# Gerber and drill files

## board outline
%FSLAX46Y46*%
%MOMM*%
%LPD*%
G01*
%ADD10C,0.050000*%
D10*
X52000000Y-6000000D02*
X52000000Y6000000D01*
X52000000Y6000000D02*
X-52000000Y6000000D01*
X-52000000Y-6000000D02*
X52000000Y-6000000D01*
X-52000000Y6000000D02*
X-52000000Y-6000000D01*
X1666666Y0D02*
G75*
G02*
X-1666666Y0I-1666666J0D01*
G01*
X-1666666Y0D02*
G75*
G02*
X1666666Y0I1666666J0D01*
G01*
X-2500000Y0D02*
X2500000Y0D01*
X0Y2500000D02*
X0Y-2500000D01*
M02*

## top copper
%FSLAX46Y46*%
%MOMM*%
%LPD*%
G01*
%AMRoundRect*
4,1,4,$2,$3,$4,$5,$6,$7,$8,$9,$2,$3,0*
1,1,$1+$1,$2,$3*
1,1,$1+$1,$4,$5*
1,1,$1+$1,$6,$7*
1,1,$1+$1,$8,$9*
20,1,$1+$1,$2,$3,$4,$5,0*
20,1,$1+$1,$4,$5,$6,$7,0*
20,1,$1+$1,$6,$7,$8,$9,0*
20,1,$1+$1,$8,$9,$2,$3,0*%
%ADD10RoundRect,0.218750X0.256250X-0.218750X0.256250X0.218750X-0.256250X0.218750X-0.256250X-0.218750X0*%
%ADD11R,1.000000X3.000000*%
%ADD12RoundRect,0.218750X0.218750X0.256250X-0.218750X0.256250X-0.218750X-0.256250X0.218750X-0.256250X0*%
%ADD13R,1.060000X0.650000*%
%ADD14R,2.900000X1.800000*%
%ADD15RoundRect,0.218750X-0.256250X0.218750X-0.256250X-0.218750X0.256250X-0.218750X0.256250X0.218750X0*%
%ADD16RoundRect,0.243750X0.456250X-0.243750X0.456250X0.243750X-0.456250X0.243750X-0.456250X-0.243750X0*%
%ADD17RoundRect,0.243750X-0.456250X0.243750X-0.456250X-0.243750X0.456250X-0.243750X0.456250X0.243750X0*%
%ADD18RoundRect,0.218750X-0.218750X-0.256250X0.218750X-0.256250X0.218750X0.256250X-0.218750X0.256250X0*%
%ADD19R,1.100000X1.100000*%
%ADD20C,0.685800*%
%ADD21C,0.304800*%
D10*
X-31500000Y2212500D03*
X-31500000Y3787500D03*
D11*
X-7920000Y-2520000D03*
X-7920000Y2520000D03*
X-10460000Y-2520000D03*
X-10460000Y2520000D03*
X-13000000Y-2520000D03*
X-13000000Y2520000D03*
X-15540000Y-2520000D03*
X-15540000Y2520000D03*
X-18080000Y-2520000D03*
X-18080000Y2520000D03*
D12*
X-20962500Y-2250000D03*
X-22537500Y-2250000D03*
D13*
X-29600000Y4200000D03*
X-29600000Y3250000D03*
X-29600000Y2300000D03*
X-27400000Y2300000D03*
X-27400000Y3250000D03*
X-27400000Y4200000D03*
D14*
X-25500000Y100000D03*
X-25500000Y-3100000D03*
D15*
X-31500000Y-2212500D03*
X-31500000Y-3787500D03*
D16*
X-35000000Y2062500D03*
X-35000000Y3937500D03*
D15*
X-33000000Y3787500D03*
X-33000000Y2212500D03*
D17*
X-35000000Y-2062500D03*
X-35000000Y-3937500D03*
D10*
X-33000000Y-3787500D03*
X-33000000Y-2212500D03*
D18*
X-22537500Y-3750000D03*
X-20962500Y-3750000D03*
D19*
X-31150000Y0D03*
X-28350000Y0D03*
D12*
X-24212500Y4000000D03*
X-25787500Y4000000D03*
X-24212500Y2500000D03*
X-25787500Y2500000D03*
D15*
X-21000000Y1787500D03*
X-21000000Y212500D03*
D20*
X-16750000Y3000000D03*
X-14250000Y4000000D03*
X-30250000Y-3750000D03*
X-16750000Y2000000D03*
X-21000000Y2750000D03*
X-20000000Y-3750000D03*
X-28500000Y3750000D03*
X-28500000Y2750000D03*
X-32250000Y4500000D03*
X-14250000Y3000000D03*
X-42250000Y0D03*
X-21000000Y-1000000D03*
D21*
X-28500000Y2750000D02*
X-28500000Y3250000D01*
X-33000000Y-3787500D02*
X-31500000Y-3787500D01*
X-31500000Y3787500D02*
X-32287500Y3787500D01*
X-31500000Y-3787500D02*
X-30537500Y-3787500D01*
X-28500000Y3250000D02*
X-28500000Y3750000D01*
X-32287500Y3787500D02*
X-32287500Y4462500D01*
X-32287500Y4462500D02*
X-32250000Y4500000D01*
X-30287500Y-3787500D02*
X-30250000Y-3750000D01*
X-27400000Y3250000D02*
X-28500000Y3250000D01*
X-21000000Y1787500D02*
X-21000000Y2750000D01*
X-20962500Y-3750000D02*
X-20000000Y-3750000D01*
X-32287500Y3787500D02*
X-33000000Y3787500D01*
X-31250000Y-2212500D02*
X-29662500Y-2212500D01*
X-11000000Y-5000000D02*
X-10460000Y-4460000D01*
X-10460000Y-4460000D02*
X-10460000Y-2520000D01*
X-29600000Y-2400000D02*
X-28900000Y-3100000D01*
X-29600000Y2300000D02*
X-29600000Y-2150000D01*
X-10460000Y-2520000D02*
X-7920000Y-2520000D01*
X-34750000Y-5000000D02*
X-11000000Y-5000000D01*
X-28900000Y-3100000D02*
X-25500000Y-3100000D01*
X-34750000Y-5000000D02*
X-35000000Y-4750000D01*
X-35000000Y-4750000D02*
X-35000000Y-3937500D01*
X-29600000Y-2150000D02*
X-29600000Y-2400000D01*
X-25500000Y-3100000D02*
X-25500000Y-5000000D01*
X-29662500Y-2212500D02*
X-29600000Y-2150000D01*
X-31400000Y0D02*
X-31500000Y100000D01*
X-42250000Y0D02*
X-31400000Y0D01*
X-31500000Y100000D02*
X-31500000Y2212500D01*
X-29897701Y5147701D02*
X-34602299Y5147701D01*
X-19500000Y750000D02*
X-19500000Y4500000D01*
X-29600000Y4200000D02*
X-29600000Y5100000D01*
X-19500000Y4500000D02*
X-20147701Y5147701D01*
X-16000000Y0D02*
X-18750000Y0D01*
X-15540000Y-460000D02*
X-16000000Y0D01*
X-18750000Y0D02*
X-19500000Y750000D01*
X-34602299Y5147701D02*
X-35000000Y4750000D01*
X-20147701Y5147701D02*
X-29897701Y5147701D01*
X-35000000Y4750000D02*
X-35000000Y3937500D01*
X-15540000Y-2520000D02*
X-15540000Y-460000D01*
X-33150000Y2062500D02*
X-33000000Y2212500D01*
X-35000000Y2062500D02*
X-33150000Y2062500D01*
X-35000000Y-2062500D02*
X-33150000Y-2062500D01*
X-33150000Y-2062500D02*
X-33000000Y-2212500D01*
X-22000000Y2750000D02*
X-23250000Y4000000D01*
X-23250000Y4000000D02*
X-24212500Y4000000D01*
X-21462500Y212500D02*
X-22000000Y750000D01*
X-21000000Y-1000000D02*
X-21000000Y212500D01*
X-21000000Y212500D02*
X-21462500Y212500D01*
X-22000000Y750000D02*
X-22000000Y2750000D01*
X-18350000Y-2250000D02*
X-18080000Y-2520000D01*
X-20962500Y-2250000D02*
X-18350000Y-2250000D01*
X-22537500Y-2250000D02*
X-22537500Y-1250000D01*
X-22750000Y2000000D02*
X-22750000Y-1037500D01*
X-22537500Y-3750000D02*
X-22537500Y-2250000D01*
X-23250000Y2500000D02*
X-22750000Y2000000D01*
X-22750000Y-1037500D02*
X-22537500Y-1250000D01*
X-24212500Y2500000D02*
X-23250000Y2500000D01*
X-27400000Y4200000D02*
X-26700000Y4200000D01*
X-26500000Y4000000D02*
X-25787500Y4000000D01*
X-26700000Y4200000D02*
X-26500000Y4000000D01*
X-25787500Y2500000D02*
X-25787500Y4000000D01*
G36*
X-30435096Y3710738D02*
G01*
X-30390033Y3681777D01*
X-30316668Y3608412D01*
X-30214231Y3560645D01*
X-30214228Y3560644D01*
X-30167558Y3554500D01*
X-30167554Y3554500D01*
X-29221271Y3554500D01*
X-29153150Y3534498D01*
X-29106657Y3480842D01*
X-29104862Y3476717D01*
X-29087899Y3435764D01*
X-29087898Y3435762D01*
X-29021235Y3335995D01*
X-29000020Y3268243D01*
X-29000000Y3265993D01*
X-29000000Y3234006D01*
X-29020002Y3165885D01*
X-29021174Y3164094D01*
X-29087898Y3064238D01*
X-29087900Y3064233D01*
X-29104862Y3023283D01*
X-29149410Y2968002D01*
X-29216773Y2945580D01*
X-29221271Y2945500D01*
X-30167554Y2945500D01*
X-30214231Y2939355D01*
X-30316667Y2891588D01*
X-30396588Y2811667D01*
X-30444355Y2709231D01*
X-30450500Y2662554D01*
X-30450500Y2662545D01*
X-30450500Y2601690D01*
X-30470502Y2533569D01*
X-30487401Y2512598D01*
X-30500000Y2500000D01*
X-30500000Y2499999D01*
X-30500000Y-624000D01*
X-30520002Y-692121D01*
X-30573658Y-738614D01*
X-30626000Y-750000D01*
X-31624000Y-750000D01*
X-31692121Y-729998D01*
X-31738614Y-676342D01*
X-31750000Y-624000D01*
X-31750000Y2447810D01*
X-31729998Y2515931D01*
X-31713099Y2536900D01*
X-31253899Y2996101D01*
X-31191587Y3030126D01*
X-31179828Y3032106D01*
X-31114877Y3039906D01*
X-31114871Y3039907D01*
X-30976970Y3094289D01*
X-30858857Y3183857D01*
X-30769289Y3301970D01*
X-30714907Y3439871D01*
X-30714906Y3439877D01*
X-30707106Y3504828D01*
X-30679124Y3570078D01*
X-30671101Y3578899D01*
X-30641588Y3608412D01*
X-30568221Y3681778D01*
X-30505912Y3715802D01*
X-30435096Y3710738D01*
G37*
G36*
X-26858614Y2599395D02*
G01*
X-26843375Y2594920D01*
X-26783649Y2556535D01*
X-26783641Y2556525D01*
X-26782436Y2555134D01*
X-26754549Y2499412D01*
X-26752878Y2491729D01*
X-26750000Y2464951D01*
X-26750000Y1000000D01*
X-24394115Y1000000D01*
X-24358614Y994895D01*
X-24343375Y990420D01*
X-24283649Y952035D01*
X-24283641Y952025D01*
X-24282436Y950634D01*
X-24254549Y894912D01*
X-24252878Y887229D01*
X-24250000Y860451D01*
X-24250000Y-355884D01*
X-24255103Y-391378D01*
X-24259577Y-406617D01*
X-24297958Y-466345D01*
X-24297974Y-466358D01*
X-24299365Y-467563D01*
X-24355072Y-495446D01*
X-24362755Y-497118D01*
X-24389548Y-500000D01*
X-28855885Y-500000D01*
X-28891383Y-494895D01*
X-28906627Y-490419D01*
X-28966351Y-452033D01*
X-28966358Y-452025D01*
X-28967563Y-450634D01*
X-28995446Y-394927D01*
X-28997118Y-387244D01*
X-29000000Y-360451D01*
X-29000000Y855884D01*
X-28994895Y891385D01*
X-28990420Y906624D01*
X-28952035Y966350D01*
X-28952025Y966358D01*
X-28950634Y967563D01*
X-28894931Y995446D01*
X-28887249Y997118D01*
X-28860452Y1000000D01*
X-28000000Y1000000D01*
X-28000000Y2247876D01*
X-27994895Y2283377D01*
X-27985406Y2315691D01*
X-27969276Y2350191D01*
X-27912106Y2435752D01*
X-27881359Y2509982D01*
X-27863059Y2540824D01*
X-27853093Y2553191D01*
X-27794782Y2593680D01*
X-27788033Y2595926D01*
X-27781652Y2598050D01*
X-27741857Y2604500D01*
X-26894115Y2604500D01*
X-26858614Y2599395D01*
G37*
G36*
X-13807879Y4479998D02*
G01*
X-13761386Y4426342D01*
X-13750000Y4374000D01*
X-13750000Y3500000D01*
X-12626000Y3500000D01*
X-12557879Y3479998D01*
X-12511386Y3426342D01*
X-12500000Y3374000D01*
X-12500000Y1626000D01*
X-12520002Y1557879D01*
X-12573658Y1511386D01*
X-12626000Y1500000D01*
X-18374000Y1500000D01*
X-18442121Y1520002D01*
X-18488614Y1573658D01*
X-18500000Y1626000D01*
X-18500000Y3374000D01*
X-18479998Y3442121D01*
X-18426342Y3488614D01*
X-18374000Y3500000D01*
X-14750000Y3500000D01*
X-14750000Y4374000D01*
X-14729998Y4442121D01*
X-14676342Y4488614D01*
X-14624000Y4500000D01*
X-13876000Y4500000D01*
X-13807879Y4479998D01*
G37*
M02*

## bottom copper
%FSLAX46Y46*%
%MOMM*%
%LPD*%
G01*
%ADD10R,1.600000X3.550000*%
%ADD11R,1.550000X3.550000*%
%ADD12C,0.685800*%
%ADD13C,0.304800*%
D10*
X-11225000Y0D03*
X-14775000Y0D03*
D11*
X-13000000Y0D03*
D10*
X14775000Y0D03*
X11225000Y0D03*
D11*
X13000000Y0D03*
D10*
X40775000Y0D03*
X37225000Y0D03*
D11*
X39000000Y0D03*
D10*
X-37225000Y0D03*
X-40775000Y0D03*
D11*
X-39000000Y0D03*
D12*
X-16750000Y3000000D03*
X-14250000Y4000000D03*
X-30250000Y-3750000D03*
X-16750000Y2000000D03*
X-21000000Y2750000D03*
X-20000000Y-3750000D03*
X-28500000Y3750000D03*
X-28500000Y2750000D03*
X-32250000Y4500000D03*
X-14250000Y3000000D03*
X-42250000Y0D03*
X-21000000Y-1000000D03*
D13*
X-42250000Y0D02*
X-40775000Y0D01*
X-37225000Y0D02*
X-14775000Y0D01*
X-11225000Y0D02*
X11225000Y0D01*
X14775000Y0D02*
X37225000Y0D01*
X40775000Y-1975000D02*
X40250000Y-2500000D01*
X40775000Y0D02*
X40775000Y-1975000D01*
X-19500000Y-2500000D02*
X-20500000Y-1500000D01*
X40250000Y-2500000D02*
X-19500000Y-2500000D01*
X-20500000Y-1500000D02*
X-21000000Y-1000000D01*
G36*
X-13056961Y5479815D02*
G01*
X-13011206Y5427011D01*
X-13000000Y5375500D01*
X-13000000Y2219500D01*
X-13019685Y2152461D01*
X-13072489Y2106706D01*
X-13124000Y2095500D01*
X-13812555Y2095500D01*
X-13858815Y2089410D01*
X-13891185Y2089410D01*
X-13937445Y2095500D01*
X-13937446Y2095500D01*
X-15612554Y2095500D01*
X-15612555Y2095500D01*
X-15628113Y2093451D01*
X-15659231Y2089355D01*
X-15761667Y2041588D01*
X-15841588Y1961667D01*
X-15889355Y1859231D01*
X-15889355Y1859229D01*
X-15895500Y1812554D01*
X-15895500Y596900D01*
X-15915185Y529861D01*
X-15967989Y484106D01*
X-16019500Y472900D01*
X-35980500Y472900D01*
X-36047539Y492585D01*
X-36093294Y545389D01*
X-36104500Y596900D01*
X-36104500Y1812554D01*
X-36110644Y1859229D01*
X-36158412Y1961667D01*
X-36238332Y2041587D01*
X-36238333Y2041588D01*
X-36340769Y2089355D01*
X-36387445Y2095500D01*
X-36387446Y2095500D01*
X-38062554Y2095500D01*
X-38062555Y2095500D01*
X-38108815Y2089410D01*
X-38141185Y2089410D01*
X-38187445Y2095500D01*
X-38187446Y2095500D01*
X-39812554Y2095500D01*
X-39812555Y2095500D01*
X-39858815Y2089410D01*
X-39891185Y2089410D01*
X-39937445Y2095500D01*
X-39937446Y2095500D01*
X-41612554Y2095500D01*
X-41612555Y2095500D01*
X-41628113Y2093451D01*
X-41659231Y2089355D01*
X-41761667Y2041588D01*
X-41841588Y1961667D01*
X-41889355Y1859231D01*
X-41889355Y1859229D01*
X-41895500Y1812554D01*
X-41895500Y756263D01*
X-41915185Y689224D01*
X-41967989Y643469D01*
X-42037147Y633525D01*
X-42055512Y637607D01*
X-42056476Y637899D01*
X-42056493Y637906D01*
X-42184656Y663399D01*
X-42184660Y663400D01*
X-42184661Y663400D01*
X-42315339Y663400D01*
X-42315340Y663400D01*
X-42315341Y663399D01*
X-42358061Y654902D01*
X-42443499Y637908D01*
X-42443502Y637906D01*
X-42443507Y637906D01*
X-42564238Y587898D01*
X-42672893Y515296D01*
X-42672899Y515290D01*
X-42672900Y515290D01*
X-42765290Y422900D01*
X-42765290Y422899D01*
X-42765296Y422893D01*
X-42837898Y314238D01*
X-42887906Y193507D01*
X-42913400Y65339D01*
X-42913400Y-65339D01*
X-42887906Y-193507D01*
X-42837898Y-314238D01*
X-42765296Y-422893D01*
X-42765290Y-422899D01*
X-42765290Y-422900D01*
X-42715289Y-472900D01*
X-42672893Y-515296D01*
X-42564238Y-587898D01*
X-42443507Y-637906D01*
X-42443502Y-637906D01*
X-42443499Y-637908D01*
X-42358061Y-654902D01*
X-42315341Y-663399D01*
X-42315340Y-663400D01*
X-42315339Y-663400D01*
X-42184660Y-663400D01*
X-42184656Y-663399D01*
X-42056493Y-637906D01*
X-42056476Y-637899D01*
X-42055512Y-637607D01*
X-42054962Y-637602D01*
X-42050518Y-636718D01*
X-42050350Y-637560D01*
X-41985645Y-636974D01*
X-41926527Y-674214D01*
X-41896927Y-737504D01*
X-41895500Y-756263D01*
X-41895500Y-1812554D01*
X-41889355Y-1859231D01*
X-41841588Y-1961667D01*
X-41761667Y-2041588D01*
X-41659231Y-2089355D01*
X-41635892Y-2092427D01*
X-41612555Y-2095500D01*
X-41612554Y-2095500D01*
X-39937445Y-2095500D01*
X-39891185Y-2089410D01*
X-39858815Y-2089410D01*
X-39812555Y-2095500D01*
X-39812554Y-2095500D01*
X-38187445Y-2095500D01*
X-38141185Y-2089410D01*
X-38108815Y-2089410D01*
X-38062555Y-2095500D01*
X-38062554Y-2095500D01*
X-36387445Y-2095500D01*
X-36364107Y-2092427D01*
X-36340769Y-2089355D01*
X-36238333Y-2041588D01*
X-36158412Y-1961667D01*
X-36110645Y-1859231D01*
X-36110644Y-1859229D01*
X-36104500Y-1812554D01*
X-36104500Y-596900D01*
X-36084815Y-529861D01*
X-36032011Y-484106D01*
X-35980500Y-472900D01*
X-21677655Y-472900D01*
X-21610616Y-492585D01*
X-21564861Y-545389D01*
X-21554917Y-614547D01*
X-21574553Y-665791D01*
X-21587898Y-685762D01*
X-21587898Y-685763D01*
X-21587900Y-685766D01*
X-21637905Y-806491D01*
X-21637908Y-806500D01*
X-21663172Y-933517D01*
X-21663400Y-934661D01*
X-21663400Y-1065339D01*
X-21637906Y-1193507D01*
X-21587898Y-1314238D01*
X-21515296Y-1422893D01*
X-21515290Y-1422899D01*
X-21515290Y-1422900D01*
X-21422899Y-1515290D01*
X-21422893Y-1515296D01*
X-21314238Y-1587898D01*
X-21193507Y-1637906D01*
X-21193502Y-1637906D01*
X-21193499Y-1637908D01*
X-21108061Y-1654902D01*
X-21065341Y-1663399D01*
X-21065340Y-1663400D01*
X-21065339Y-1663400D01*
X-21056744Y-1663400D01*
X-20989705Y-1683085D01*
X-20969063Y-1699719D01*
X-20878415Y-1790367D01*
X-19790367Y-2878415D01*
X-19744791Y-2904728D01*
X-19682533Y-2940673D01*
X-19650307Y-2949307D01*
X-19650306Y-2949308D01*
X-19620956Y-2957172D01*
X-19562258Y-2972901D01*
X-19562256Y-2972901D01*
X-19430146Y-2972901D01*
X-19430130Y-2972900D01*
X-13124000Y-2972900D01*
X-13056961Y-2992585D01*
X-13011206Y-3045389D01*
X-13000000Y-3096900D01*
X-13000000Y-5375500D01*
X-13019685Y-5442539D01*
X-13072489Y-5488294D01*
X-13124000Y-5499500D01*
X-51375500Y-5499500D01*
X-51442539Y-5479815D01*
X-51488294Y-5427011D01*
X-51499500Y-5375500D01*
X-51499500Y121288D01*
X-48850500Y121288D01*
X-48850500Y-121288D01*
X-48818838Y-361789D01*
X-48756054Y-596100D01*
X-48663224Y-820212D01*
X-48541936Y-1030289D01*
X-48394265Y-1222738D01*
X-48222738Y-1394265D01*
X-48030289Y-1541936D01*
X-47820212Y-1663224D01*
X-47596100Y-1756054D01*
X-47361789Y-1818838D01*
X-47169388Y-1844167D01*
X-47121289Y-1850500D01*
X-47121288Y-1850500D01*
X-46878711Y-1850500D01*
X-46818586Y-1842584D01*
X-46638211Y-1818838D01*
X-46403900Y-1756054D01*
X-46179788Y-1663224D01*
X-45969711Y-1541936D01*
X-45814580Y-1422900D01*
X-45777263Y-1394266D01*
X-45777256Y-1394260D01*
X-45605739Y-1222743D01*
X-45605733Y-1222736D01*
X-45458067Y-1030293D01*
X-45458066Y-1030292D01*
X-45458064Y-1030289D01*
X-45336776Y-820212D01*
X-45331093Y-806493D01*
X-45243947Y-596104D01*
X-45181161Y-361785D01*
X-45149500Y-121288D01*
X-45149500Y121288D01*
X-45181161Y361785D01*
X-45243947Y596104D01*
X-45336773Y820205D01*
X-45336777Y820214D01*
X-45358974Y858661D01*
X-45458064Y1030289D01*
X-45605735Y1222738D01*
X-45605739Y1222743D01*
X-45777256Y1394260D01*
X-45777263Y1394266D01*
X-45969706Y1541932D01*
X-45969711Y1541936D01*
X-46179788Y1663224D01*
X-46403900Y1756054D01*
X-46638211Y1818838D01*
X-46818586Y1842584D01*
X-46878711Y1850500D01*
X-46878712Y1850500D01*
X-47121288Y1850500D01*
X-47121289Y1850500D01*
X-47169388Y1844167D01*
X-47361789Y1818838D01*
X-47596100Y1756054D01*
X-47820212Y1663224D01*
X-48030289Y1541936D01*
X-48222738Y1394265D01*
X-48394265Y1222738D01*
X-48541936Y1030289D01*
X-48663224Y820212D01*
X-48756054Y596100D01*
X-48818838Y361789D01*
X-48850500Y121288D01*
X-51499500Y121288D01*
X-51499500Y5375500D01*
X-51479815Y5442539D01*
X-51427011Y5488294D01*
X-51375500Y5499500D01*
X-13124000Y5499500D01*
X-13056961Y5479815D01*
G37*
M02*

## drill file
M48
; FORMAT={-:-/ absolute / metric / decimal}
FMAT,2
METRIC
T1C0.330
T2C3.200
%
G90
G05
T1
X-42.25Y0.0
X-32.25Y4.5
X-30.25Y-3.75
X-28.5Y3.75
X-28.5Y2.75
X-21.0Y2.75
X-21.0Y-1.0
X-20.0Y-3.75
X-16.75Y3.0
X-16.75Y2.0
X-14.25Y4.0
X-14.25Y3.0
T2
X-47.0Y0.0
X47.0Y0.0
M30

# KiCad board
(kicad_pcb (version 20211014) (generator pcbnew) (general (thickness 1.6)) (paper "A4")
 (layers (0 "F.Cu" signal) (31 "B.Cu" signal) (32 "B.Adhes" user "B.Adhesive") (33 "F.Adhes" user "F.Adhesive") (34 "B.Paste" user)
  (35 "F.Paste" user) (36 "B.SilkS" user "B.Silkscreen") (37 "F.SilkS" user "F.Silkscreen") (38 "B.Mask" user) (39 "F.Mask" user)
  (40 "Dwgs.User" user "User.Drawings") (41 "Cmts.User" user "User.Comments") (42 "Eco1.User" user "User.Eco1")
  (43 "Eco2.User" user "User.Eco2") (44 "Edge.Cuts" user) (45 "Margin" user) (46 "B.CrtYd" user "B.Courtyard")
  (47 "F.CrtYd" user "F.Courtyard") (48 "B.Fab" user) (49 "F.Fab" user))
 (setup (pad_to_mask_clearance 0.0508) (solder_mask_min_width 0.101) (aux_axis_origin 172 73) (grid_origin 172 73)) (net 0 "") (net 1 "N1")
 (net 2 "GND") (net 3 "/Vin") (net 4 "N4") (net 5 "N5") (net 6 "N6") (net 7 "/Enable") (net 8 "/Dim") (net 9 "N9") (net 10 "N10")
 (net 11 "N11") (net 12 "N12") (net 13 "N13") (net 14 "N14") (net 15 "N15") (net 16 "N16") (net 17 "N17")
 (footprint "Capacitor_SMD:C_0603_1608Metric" (layer "F.Cu") (at -31.5 -3 90)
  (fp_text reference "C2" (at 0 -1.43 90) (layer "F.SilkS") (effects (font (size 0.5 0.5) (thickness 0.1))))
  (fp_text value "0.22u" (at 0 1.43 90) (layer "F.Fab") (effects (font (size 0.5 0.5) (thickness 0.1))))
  (pad "1" smd roundrect locked (at -0.7875 0 90) (size 0.875 0.95) (layers "F.Cu" "F.Paste" "F.Mask") (roundrect_rratio 0.25) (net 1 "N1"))
  (pad "2" smd roundrect locked (at 0.7875 0 90) (size 0.875 0.95) (layers "F.Cu" "F.Paste" "F.Mask") (roundrect_rratio 0.25) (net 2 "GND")))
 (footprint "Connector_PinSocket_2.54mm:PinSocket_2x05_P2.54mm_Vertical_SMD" (layer "F.Cu") (at -13 0 -90)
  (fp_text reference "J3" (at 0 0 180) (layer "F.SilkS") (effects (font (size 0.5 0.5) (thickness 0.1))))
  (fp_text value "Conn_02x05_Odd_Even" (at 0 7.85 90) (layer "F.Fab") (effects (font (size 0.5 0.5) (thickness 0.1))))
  (pad "1" smd rect locked (at 2.52 -5.08 270) (size 3 1) (layers "F.Cu" "F.Paste" "F.Mask") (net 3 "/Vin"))
  (pad "2" smd rect locked (at -2.52 -5.08 270) (size 3 1) (layers "F.Cu" "F.Paste" "F.Mask") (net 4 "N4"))
  (pad "3" smd rect locked (at 2.52 -2.54 270) (size 3 1) (layers "F.Cu" "F.Paste" "F.Mask") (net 3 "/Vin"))
  (pad "4" smd rect locked (at -2.52 -2.54 270) (size 3 1) (layers "F.Cu" "F.Paste" "F.Mask") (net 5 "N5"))
  (pad "5" smd rect locked (at 2.52 0 270) (size 3 1) (layers "F.Cu" "F.Paste" "F.Mask") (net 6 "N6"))
  (pad "6" smd rect locked (at -2.52 0 270) (size 3 1) (layers "F.Cu" "F.Paste" "F.Mask") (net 2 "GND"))
  (pad "7" smd rect locked (at 2.52 2.54 270) (size 3 1) (layers "F.Cu" "F.Paste" "F.Mask") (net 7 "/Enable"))
  (pad "8" smd rect locked (at -2.52 2.54 270) (size 3 1) (layers "F.Cu" "F.Paste" "F.Mask") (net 2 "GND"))
  (pad "9" smd rect locked (at 2.52 5.08 270) (size 3 1) (layers "F.Cu" "F.Paste" "F.Mask") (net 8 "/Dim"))
  (pad "10" smd rect locked (at -2.52 5.08 270) (size 3 1) (layers "F.Cu" "F.Paste" "F.Mask") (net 2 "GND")))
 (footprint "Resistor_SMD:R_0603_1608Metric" (layer "F.Cu") (at -21.75 2.25 180)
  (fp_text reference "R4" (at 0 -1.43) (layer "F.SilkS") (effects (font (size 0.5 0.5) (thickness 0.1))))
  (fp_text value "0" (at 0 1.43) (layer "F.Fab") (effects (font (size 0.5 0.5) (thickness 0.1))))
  (pad "1" smd roundrect locked (at -0.7875 0 180) (size 0.875 0.95) (layers "F.Cu" "F.Paste" "F.Mask") (roundrect_rratio 0.25)
   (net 8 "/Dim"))
  (pad "2" smd roundrect locked (at 0.7875 0 180) (size 0.875 0.95) (layers "F.Cu" "F.Paste" "F.Mask") (roundrect_rratio 0.25) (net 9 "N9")))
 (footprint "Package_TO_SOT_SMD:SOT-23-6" (layer "F.Cu") (at -28.5 -3.25)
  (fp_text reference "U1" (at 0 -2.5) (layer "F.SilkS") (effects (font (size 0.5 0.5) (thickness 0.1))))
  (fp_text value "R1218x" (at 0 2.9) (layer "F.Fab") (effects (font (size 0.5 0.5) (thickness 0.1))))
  (pad "1" smd rect locked (at -1.1 -0.95) (size 1.06 0.65) (layers "F.Cu" "F.Paste" "F.Mask") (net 7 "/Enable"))
  (pad "2" smd rect locked (at -1.1 0) (size 1.06 0.65) (layers "F.Cu" "F.Paste" "F.Mask") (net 1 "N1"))
  (pad "3" smd rect locked (at -1.1 0.95) (size 1.06 0.65) (layers "F.Cu" "F.Paste" "F.Mask") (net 3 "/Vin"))
  (pad "4" smd rect locked (at 1.1 0.95) (size 1.06 0.65) (layers "F.Cu" "F.Paste" "F.Mask") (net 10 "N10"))
  (pad "5" smd rect locked (at 1.1 0) (size 1.06 0.65) (layers "F.Cu" "F.Paste" "F.Mask") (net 2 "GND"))
  (pad "6" smd rect locked (at 1.1 -0.95) (size 1.06 0.65) (layers "F.Cu" "F.Paste" "F.Mask") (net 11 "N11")))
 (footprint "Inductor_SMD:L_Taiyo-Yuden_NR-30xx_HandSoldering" (layer "F.Cu") (at -25.5 1.5 -90)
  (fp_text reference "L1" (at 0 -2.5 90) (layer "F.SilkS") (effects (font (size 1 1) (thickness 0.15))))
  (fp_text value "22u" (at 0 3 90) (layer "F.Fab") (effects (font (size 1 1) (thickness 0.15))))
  (pad "1" smd rect locked (at -1.6 0 270) (size 1.8 2.9) (layers "F.Cu" "F.Paste" "F.Mask") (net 10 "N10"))
  (pad "2" smd rect locked (at 1.6 0 270) (size 1.8 2.9) (layers "F.Cu" "F.Paste" "F.Mask") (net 3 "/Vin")))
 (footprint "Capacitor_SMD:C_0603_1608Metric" (layer "F.Cu") (at -31.5 3 -90)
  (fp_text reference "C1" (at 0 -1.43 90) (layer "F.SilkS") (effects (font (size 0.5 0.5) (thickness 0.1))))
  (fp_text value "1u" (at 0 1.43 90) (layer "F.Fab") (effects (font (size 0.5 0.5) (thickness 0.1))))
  (pad "1" smd roundrect locked (at -0.7875 0 270) (size 0.875 0.95) (layers "F.Cu" "F.Paste" "F.Mask") (roundrect_rratio 0.25)
   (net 3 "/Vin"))
  (pad "2" smd roundrect locked (at 0.7875 0 270) (size 0.875 0.95) (layers "F.Cu" "F.Paste" "F.Mask") (roundrect_rratio 0.25) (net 2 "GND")))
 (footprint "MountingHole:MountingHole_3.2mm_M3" (layer "F.Cu") (at 47 0)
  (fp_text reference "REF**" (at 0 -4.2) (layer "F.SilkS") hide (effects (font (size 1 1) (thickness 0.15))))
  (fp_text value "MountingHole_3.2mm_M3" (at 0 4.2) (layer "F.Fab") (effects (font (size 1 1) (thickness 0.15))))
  (pad "" np_thru_hole circle locked (at 0 0) (size 3.2 3.2) (drill 3.2) (layers *.Cu *.Mask)))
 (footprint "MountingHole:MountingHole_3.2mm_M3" (layer "F.Cu") (at -47 0)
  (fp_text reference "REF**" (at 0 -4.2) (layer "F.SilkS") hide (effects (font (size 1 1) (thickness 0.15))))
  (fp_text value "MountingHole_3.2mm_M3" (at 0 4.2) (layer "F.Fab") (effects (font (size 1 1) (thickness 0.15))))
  (pad "" np_thru_hole circle locked (at 0 0) (size 3.2 3.2) (drill 3.2) (layers *.Cu *.Mask)))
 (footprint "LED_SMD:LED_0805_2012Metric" (layer "F.Cu") (at -35 -3 90)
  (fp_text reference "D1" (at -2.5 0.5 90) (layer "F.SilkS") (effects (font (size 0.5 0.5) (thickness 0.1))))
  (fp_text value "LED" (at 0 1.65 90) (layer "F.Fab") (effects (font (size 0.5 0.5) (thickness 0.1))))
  (pad "1" smd roundrect locked (at -0.9375 0 90) (size 0.975 1.4) (layers "F.Cu" "F.Paste" "F.Mask") (roundrect_rratio 0.25) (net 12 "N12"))
  (pad "2" smd roundrect locked (at 0.9375 0 90) (size 0.975 1.4) (layers "F.Cu" "F.Paste" "F.Mask") (roundrect_rratio 0.25)
   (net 7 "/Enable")))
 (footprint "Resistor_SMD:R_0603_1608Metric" (layer "F.Cu") (at -33 -3 -90)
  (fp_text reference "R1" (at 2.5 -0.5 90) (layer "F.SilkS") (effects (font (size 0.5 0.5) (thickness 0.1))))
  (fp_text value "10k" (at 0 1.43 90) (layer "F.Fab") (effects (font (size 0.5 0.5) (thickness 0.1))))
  (pad "1" smd roundrect locked (at -0.7875 0 270) (size 0.875 0.95) (layers "F.Cu" "F.Paste" "F.Mask") (roundrect_rratio 0.25)
   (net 2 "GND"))
  (pad "2" smd roundrect locked (at 0.7875 0 270) (size 0.875 0.95) (layers "F.Cu" "F.Paste" "F.Mask") (roundrect_rratio 0.25)
   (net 12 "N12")))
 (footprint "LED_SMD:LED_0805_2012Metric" (layer "F.Cu") (at -35 3 -90)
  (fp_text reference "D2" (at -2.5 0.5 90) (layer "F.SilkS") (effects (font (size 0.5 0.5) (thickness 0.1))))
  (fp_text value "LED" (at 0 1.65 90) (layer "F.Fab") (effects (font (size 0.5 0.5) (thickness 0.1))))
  (pad "1" smd roundrect locked (at -0.9375 0 270) (size 0.975 1.4) (layers "F.Cu" "F.Paste" "F.Mask") (roundrect_rratio 0.25)
   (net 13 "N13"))
  (pad "2" smd roundrect locked (at 0.9375 0 270) (size 0.975 1.4) (layers "F.Cu" "F.Paste" "F.Mask") (roundrect_rratio 0.25) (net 3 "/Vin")))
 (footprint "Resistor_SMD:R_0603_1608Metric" (layer "F.Cu") (at -33 3 90)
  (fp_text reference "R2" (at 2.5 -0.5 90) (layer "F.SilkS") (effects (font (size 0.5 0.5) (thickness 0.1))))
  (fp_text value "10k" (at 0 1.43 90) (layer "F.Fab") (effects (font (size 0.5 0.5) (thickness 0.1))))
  (pad "1" smd roundrect locked (at -0.7875 0 90) (size 0.875 0.95) (layers "F.Cu" "F.Paste" "F.Mask") (roundrect_rratio 0.25) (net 2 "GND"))
  (pad "2" smd roundrect locked (at 0.7875 0 90) (size 0.875 0.95) (layers "F.Cu" "F.Paste" "F.Mask") (roundrect_rratio 0.25) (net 13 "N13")))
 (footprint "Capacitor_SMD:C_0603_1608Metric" (layer "F.Cu") (at -21.75 3.75)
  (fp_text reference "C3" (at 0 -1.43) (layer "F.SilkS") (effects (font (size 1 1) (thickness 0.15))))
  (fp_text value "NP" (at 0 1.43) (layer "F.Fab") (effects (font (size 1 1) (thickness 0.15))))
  (pad "1" smd roundrect locked (at -0.7875 0) (size 0.875 0.95) (layers "F.Cu" "F.Paste" "F.Mask") (roundrect_rratio 0.25) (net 9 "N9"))
  (pad "2" smd roundrect locked (at 0.7875 0) (size 0.875 0.95) (layers "F.Cu" "F.Paste" "F.Mask") (roundrect_rratio 0.25) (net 2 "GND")))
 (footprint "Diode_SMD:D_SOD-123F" (layer "F.Cu") (at -29.75 0)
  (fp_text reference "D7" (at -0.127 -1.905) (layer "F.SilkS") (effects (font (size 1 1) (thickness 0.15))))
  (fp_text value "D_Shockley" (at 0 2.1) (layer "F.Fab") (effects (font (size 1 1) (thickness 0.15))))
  (pad "1" smd rect locked (at -1.4 0) (size 1.1 1.1) (layers "F.Cu" "F.Paste" "F.Mask") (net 1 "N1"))
  (pad "2" smd rect locked (at 1.4 0) (size 1.1 1.1) (layers "F.Cu" "F.Paste" "F.Mask") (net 10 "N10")))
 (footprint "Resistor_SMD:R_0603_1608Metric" (layer "F.Cu") (at -25 -4 180)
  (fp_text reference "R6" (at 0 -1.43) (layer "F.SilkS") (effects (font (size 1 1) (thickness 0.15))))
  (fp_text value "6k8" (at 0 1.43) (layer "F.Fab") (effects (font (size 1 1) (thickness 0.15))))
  (pad "1" smd roundrect locked (at -0.7875 0 180) (size 0.875 0.95) (layers "F.Cu" "F.Paste" "F.Mask") (roundrect_rratio 0.25)
   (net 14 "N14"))
  (pad "2" smd roundrect locked (at 0.7875 0 180) (size 0.875 0.95) (layers "F.Cu" "F.Paste" "F.Mask") (roundrect_rratio 0.25)
   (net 11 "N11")))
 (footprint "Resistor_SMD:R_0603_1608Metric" (layer "F.Cu") (at -25 -2.5 180)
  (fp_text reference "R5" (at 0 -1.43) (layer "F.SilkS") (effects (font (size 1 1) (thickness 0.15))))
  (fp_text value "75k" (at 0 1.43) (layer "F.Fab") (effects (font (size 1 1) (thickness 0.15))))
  (pad "1" smd roundrect locked (at -0.7875 0 180) (size 0.875 0.95) (layers "F.Cu" "F.Paste" "F.Mask") (roundrect_rratio 0.25) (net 9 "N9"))
  (pad "2" smd roundrect locked (at 0.7875 0 180) (size 0.875 0.95) (layers "F.Cu" "F.Paste" "F.Mask") (roundrect_rratio 0.25)
   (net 11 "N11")))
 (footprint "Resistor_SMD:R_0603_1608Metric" (layer "F.Cu") (at -21 -1 -90)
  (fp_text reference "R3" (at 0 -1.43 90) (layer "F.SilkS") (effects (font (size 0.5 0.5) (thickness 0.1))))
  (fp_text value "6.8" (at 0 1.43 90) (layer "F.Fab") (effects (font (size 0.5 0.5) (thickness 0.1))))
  (pad "1" smd roundrect locked (at -0.7875 0 270) (size 0.875 0.95) (layers "F.Cu" "F.Paste" "F.Mask") (roundrect_rratio 0.25)
   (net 2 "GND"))
  (pad "2" smd roundrect locked (at 0.7875 0 270) (size 0.875 0.95) (layers "F.Cu" "F.Paste" "F.Mask") (roundrect_rratio 0.25)
   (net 14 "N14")))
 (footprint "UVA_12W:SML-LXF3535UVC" (layer "B.Cu") (at -13 0 180)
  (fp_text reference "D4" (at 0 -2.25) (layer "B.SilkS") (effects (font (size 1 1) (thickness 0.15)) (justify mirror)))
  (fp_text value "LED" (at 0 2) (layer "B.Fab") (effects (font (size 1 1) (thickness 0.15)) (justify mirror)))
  (pad "1" smd rect locked (at -1.775 0 180) (size 1.6 3.55) (layers "B.Cu" "B.Paste" "B.Mask") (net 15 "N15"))
  (pad "2" smd rect locked (at 1.775 0 180) (size 1.6 3.55) (layers "B.Cu" "B.Paste" "B.Mask") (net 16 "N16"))
  (pad "3" smd rect locked (at 0 0 180) (size 1.55 3.55) (layers "B.Cu" "B.Paste" "B.Mask")))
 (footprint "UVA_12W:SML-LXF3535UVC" (layer "B.Cu") (at 13 0 180)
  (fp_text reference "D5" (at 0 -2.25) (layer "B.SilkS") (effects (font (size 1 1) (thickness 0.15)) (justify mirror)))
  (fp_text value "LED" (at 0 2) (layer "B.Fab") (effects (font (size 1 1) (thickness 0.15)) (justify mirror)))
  (pad "1" smd rect locked (at -1.775 0 180) (size 1.6 3.55) (layers "B.Cu" "B.Paste" "B.Mask") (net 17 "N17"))
  (pad "2" smd rect locked (at 1.775 0 180) (size 1.6 3.55) (layers "B.Cu" "B.Paste" "B.Mask") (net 15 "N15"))
  (pad "3" smd rect locked (at 0 0 180) (size 1.55 3.55) (layers "B.Cu" "B.Paste" "B.Mask")))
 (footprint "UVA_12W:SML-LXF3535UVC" (layer "B.Cu") (at 39 0 180)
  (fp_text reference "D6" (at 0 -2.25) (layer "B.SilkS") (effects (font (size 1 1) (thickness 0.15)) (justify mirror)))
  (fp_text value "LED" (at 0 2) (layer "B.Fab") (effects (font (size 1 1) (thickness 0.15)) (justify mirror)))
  (pad "1" smd rect locked (at -1.775 0 180) (size 1.6 3.55) (layers "B.Cu" "B.Paste" "B.Mask") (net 14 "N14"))
  (pad "2" smd rect locked (at 1.775 0 180) (size 1.6 3.55) (layers "B.Cu" "B.Paste" "B.Mask") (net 17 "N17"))
  (pad "3" smd rect locked (at 0 0 180) (size 1.55 3.55) (layers "B.Cu" "B.Paste" "B.Mask")))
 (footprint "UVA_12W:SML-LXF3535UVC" (layer "B.Cu") (at -39 0 180)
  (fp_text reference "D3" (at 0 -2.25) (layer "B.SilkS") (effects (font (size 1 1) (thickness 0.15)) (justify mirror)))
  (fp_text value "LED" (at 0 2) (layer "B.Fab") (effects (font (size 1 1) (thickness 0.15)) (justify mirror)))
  (pad "1" smd rect locked (at -1.775 0 180) (size 1.6 3.55) (layers "B.Cu" "B.Paste" "B.Mask") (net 16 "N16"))
  (pad "2" smd rect locked (at 1.775 0 180) (size 1.6 3.55) (layers "B.Cu" "B.Paste" "B.Mask") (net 1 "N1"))
  (pad "3" smd rect locked (at 0 0 180) (size 1.55 3.55) (layers "B.Cu" "B.Paste" "B.Mask")))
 (gr_line (start 52 6) (end 52 -6) (layer "Edge.Cuts") (width 0.05))
 (gr_line (start 52 -6) (end -52 -6) (layer "Edge.Cuts") (width 0.05))
 (gr_line (start -52 6) (end 52 6) (layer "Edge.Cuts") (width 0.05))
 (gr_line (start -52 -6) (end -52 6) (layer "Edge.Cuts") (width 0.05))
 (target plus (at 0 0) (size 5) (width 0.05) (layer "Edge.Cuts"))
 (segment (start -28.5 -2.75) (end -28.5 -3.25) (width 0.3048) (layer "F.Cu") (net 2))
 (segment (start -33 3.7875) (end -31.5 3.7875) (width 0.3048) (layer "F.Cu") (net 2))
 (segment (start -31.5 -3.7875) (end -32.2875 -3.7875) (width 0.3048) (layer "F.Cu") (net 2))
 (segment (start -31.5 3.7875) (end -30.5375 3.7875) (width 0.3048) (layer "F.Cu") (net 2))
 (segment (start -28.5 -3.25) (end -28.5 -3.75) (width 0.3048) (layer "F.Cu") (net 2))
 (segment (start -32.2875 -3.7875) (end -32.2875 -4.4625) (width 0.3048) (layer "F.Cu") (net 2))
 (segment (start -32.2875 -4.4625) (end -32.25 -4.5) (width 0.3048) (layer "F.Cu") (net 2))
 (segment (start -30.2875 3.7875) (end -30.25 3.75) (width 0.3048) (layer "F.Cu") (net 2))
 (segment (start -27.4 -3.25) (end -28.5 -3.25) (width 0.3048) (layer "F.Cu") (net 2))
 (segment (start -21 -1.7875) (end -21 -2.75) (width 0.3048) (layer "F.Cu") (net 2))
 (segment (start -20.9625 3.75) (end -20 3.75) (width 0.3048) (layer "F.Cu") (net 2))
 (segment (start -32.2875 -3.7875) (end -33 -3.7875) (width 0.3048) (layer "F.Cu") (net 2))
 (via (at -16.75 -3) (size 0.6858) (drill 0.3302) (layers "F.Cu" "B.Cu") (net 2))
 (via (at -14.25 -4) (size 0.6858) (drill 0.3302) (layers "F.Cu" "B.Cu") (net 2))
 (via (at -30.25 3.75) (size 0.6858) (drill 0.3302) (layers "F.Cu" "B.Cu") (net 2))
 (via (at -16.75 -2) (size 0.6858) (drill 0.3302) (layers "F.Cu" "B.Cu") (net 2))
 (via (at -21 -2.75) (size 0.6858) (drill 0.3302) (layers "F.Cu" "B.Cu") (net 2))
 (via (at -20 3.75) (size 0.6858) (drill 0.3302) (layers "F.Cu" "B.Cu") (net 2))
 (via (at -28.5 -3.75) (size 0.6858) (drill 0.3302) (layers "F.Cu" "B.Cu") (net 2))
 (via (at -28.5 -2.75) (size 0.6858) (drill 0.3302) (layers "F.Cu" "B.Cu") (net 2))
 (via (at -32.25 -4.5) (size 0.6858) (drill 0.3302) (layers "F.Cu" "B.Cu") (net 2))
 (via (at -14.25 -3) (size 0.6858) (drill 0.3302) (layers "F.Cu" "B.Cu") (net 2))
 (segment (start -31.25 2.2125) (end -29.6625 2.2125) (width 0.3048) (layer "F.Cu") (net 3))
 (segment (start -11 5) (end -10.46 4.46) (width 0.3048) (layer "F.Cu") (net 3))
 (segment (start -10.46 4.46) (end -10.46 2.52) (width 0.3048) (layer "F.Cu") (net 3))
 (segment (start -29.6 2.4) (end -28.9 3.1) (width 0.3048) (layer "F.Cu") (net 3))
 (segment (start -29.6 -2.3) (end -29.6 2.15) (width 0.3048) (layer "F.Cu") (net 3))
 (segment (start -10.46 2.52) (end -7.92 2.52) (width 0.3048) (layer "F.Cu") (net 3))
 (segment (start -34.75 5) (end -11 5) (width 0.3048) (layer "F.Cu") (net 3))
 (segment (start -28.9 3.1) (end -25.5 3.1) (width 0.3048) (layer "F.Cu") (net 3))
 (segment (start -34.75 5) (end -35 4.75) (width 0.3048) (layer "F.Cu") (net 3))
 (segment (start -35 4.75) (end -35 3.9375) (width 0.3048) (layer "F.Cu") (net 3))
 (segment (start -29.6 2.15) (end -29.6 2.4) (width 0.3048) (layer "F.Cu") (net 3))
 (segment (start -25.5 3.1) (end -25.5 5) (width 0.3048) (layer "F.Cu") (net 3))
 (segment (start -29.6625 2.2125) (end -29.6 2.15) (width 0.3048) (layer "F.Cu") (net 3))
 (segment (start -31.4 0) (end -31.5 -0.1) (width 0.3048) (layer "F.Cu") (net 1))
 (segment (start -42.25 0) (end -31.4 0) (width 0.3048) (layer "F.Cu") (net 1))
 (segment (start -31.5 -0.1) (end -31.5 -2.2125) (width 0.3048) (layer "F.Cu") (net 1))
 (via (at -42.25 0) (size 0.6858) (drill 0.3302) (layers "F.Cu" "B.Cu") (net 1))
 (segment (start -42.25 0) (end -40.775 0) (width 0.3048) (layer "B.Cu") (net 1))
 (segment (start -29.897701 -5.147701) (end -34.602299 -5.147701) (width 0.3048) (layer "F.Cu") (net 7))
 (segment (start -19.5 -0.75) (end -19.5 -4.5) (width 0.3048) (layer "F.Cu") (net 7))
 (segment (start -29.6 -4.2) (end -29.6 -5.1) (width 0.3048) (layer "F.Cu") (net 7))
 (segment (start -19.5 -4.5) (end -20.147701 -5.147701) (width 0.3048) (layer "F.Cu") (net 7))
 (segment (start -16 0) (end -18.75 0) (width 0.3048) (layer "F.Cu") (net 7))
 (segment (start -15.54 0.46) (end -16 0) (width 0.3048) (layer "F.Cu") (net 7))
 (segment (start -18.75 0) (end -19.5 -0.75) (width 0.3048) (layer "F.Cu") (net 7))
 (segment (start -34.602299 -5.147701) (end -35 -4.75) (width 0.3048) (layer "F.Cu") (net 7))
 (segment (start -20.147701 -5.147701) (end -29.897701 -5.147701) (width 0.3048) (layer "F.Cu") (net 7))
 (segment (start -35 -4.75) (end -35 -3.9375) (width 0.3048) (layer "F.Cu") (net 7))
 (segment (start -15.54 2.52) (end -15.54 0.46) (width 0.3048) (layer "F.Cu") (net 7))
 (segment (start -33.15 -2.0625) (end -33 -2.2125) (width 0.3048) (layer "F.Cu") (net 12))
 (segment (start -35 -2.0625) (end -33.15 -2.0625) (width 0.3048) (layer "F.Cu") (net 12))
 (segment (start -35 2.0625) (end -33.15 2.0625) (width 0.3048) (layer "F.Cu") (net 13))
 (segment (start -33.15 2.0625) (end -33 2.2125) (width 0.3048) (layer "F.Cu") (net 13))
 (segment (start -37.225 0) (end -14.775 0) (width 0.3048) (layer "B.Cu") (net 16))
 (segment (start -11.225 0) (end 11.225 0) (width 0.3048) (layer "B.Cu") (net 15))
 (segment (start 14.775 0) (end 37.225 0) (width 0.3048) (layer "B.Cu") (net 17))
 (segment (start -22 -2.75) (end -23.25 -4) (width 0.3048) (layer "F.Cu") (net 14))
 (segment (start -23.25 -4) (end -24.2125 -4) (width 0.3048) (layer "F.Cu") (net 14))
 (segment (start -21.4625 -0.2125) (end -22 -0.75) (width 0.3048) (layer "F.Cu") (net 14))
 (segment (start -21 1) (end -21 -0.2125) (width 0.3048) (layer "F.Cu") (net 14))
 (segment (start -21 -0.2125) (end -21.4625 -0.2125) (width 0.3048) (layer "F.Cu") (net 14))
 (segment (start -22 -0.75) (end -22 -2.75) (width 0.3048) (layer "F.Cu") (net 14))
 (via (at -21 1) (size 0.6858) (drill 0.3302) (layers "F.Cu" "B.Cu") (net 14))
 (segment (start 40.775 1.975) (end 40.25 2.5) (width 0.3048) (layer "B.Cu") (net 14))
 (segment (start 40.775 0) (end 40.775 1.975) (width 0.3048) (layer "B.Cu") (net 14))
 (segment (start -19.5 2.5) (end -20.5 1.5) (width 0.3048) (layer "B.Cu") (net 14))
 (segment (start 40.25 2.5) (end -19.5 2.5) (width 0.3048) (layer "B.Cu") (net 14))
 (segment (start -20.5 1.5) (end -21 1) (width 0.3048) (layer "B.Cu") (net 14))
 (segment (start -18.35 2.25) (end -18.08 2.52) (width 0.3048) (layer "F.Cu") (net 8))
 (segment (start -20.9625 2.25) (end -18.35 2.25) (width 0.3048) (layer "F.Cu") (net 8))
 (segment (start -22.5375 2.25) (end -22.5375 1.25) (width 0.3048) (layer "F.Cu") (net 9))
 (segment (start -22.75 -2) (end -22.75 1.0375) (width 0.3048) (layer "F.Cu") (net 9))
 (segment (start -22.5375 3.75) (end -22.5375 2.25) (width 0.3048) (layer "F.Cu") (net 9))
 (segment (start -23.25 -2.5) (end -22.75 -2) (width 0.3048) (layer "F.Cu") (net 9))
 (segment (start -22.75 1.0375) (end -22.5375 1.25) (width 0.3048) (layer "F.Cu") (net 9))
 (segment (start -24.2125 -2.5) (end -23.25 -2.5) (width 0.3048) (layer "F.Cu") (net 9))
 (segment (start -27.4 -4.2) (end -26.7 -4.2) (width 0.3048) (layer "F.Cu") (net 11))
 (segment (start -26.5 -4) (end -25.7875 -4) (width 0.3048) (layer "F.Cu") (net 11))
 (segment (start -26.7 -4.2) (end -26.5 -4) (width 0.3048) (layer "F.Cu") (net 11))
 (segment (start -25.7875 -2.5) (end -25.7875 -4) (width 0.3048) (layer "F.Cu") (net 11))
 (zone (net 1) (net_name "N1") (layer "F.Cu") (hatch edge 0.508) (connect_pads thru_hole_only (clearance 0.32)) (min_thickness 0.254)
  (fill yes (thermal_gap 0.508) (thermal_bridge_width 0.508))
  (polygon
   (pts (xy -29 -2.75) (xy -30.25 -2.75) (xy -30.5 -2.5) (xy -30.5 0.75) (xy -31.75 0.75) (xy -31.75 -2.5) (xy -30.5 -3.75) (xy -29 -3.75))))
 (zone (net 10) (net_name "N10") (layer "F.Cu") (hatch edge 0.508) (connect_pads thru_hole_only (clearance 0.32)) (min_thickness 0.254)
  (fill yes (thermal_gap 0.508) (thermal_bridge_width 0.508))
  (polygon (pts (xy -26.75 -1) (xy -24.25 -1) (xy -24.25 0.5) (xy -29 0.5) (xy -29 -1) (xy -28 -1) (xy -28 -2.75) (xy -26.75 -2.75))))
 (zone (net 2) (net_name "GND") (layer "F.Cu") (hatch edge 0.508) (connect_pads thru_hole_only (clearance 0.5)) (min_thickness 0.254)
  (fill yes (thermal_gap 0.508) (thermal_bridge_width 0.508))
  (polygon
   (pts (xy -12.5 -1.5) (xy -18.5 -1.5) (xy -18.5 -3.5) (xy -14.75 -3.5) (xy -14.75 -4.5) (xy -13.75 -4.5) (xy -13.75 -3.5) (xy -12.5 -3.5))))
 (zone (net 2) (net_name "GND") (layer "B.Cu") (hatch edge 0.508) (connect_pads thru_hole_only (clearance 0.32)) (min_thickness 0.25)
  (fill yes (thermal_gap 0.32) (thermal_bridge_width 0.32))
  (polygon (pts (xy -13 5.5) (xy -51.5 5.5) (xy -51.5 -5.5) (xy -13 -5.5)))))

